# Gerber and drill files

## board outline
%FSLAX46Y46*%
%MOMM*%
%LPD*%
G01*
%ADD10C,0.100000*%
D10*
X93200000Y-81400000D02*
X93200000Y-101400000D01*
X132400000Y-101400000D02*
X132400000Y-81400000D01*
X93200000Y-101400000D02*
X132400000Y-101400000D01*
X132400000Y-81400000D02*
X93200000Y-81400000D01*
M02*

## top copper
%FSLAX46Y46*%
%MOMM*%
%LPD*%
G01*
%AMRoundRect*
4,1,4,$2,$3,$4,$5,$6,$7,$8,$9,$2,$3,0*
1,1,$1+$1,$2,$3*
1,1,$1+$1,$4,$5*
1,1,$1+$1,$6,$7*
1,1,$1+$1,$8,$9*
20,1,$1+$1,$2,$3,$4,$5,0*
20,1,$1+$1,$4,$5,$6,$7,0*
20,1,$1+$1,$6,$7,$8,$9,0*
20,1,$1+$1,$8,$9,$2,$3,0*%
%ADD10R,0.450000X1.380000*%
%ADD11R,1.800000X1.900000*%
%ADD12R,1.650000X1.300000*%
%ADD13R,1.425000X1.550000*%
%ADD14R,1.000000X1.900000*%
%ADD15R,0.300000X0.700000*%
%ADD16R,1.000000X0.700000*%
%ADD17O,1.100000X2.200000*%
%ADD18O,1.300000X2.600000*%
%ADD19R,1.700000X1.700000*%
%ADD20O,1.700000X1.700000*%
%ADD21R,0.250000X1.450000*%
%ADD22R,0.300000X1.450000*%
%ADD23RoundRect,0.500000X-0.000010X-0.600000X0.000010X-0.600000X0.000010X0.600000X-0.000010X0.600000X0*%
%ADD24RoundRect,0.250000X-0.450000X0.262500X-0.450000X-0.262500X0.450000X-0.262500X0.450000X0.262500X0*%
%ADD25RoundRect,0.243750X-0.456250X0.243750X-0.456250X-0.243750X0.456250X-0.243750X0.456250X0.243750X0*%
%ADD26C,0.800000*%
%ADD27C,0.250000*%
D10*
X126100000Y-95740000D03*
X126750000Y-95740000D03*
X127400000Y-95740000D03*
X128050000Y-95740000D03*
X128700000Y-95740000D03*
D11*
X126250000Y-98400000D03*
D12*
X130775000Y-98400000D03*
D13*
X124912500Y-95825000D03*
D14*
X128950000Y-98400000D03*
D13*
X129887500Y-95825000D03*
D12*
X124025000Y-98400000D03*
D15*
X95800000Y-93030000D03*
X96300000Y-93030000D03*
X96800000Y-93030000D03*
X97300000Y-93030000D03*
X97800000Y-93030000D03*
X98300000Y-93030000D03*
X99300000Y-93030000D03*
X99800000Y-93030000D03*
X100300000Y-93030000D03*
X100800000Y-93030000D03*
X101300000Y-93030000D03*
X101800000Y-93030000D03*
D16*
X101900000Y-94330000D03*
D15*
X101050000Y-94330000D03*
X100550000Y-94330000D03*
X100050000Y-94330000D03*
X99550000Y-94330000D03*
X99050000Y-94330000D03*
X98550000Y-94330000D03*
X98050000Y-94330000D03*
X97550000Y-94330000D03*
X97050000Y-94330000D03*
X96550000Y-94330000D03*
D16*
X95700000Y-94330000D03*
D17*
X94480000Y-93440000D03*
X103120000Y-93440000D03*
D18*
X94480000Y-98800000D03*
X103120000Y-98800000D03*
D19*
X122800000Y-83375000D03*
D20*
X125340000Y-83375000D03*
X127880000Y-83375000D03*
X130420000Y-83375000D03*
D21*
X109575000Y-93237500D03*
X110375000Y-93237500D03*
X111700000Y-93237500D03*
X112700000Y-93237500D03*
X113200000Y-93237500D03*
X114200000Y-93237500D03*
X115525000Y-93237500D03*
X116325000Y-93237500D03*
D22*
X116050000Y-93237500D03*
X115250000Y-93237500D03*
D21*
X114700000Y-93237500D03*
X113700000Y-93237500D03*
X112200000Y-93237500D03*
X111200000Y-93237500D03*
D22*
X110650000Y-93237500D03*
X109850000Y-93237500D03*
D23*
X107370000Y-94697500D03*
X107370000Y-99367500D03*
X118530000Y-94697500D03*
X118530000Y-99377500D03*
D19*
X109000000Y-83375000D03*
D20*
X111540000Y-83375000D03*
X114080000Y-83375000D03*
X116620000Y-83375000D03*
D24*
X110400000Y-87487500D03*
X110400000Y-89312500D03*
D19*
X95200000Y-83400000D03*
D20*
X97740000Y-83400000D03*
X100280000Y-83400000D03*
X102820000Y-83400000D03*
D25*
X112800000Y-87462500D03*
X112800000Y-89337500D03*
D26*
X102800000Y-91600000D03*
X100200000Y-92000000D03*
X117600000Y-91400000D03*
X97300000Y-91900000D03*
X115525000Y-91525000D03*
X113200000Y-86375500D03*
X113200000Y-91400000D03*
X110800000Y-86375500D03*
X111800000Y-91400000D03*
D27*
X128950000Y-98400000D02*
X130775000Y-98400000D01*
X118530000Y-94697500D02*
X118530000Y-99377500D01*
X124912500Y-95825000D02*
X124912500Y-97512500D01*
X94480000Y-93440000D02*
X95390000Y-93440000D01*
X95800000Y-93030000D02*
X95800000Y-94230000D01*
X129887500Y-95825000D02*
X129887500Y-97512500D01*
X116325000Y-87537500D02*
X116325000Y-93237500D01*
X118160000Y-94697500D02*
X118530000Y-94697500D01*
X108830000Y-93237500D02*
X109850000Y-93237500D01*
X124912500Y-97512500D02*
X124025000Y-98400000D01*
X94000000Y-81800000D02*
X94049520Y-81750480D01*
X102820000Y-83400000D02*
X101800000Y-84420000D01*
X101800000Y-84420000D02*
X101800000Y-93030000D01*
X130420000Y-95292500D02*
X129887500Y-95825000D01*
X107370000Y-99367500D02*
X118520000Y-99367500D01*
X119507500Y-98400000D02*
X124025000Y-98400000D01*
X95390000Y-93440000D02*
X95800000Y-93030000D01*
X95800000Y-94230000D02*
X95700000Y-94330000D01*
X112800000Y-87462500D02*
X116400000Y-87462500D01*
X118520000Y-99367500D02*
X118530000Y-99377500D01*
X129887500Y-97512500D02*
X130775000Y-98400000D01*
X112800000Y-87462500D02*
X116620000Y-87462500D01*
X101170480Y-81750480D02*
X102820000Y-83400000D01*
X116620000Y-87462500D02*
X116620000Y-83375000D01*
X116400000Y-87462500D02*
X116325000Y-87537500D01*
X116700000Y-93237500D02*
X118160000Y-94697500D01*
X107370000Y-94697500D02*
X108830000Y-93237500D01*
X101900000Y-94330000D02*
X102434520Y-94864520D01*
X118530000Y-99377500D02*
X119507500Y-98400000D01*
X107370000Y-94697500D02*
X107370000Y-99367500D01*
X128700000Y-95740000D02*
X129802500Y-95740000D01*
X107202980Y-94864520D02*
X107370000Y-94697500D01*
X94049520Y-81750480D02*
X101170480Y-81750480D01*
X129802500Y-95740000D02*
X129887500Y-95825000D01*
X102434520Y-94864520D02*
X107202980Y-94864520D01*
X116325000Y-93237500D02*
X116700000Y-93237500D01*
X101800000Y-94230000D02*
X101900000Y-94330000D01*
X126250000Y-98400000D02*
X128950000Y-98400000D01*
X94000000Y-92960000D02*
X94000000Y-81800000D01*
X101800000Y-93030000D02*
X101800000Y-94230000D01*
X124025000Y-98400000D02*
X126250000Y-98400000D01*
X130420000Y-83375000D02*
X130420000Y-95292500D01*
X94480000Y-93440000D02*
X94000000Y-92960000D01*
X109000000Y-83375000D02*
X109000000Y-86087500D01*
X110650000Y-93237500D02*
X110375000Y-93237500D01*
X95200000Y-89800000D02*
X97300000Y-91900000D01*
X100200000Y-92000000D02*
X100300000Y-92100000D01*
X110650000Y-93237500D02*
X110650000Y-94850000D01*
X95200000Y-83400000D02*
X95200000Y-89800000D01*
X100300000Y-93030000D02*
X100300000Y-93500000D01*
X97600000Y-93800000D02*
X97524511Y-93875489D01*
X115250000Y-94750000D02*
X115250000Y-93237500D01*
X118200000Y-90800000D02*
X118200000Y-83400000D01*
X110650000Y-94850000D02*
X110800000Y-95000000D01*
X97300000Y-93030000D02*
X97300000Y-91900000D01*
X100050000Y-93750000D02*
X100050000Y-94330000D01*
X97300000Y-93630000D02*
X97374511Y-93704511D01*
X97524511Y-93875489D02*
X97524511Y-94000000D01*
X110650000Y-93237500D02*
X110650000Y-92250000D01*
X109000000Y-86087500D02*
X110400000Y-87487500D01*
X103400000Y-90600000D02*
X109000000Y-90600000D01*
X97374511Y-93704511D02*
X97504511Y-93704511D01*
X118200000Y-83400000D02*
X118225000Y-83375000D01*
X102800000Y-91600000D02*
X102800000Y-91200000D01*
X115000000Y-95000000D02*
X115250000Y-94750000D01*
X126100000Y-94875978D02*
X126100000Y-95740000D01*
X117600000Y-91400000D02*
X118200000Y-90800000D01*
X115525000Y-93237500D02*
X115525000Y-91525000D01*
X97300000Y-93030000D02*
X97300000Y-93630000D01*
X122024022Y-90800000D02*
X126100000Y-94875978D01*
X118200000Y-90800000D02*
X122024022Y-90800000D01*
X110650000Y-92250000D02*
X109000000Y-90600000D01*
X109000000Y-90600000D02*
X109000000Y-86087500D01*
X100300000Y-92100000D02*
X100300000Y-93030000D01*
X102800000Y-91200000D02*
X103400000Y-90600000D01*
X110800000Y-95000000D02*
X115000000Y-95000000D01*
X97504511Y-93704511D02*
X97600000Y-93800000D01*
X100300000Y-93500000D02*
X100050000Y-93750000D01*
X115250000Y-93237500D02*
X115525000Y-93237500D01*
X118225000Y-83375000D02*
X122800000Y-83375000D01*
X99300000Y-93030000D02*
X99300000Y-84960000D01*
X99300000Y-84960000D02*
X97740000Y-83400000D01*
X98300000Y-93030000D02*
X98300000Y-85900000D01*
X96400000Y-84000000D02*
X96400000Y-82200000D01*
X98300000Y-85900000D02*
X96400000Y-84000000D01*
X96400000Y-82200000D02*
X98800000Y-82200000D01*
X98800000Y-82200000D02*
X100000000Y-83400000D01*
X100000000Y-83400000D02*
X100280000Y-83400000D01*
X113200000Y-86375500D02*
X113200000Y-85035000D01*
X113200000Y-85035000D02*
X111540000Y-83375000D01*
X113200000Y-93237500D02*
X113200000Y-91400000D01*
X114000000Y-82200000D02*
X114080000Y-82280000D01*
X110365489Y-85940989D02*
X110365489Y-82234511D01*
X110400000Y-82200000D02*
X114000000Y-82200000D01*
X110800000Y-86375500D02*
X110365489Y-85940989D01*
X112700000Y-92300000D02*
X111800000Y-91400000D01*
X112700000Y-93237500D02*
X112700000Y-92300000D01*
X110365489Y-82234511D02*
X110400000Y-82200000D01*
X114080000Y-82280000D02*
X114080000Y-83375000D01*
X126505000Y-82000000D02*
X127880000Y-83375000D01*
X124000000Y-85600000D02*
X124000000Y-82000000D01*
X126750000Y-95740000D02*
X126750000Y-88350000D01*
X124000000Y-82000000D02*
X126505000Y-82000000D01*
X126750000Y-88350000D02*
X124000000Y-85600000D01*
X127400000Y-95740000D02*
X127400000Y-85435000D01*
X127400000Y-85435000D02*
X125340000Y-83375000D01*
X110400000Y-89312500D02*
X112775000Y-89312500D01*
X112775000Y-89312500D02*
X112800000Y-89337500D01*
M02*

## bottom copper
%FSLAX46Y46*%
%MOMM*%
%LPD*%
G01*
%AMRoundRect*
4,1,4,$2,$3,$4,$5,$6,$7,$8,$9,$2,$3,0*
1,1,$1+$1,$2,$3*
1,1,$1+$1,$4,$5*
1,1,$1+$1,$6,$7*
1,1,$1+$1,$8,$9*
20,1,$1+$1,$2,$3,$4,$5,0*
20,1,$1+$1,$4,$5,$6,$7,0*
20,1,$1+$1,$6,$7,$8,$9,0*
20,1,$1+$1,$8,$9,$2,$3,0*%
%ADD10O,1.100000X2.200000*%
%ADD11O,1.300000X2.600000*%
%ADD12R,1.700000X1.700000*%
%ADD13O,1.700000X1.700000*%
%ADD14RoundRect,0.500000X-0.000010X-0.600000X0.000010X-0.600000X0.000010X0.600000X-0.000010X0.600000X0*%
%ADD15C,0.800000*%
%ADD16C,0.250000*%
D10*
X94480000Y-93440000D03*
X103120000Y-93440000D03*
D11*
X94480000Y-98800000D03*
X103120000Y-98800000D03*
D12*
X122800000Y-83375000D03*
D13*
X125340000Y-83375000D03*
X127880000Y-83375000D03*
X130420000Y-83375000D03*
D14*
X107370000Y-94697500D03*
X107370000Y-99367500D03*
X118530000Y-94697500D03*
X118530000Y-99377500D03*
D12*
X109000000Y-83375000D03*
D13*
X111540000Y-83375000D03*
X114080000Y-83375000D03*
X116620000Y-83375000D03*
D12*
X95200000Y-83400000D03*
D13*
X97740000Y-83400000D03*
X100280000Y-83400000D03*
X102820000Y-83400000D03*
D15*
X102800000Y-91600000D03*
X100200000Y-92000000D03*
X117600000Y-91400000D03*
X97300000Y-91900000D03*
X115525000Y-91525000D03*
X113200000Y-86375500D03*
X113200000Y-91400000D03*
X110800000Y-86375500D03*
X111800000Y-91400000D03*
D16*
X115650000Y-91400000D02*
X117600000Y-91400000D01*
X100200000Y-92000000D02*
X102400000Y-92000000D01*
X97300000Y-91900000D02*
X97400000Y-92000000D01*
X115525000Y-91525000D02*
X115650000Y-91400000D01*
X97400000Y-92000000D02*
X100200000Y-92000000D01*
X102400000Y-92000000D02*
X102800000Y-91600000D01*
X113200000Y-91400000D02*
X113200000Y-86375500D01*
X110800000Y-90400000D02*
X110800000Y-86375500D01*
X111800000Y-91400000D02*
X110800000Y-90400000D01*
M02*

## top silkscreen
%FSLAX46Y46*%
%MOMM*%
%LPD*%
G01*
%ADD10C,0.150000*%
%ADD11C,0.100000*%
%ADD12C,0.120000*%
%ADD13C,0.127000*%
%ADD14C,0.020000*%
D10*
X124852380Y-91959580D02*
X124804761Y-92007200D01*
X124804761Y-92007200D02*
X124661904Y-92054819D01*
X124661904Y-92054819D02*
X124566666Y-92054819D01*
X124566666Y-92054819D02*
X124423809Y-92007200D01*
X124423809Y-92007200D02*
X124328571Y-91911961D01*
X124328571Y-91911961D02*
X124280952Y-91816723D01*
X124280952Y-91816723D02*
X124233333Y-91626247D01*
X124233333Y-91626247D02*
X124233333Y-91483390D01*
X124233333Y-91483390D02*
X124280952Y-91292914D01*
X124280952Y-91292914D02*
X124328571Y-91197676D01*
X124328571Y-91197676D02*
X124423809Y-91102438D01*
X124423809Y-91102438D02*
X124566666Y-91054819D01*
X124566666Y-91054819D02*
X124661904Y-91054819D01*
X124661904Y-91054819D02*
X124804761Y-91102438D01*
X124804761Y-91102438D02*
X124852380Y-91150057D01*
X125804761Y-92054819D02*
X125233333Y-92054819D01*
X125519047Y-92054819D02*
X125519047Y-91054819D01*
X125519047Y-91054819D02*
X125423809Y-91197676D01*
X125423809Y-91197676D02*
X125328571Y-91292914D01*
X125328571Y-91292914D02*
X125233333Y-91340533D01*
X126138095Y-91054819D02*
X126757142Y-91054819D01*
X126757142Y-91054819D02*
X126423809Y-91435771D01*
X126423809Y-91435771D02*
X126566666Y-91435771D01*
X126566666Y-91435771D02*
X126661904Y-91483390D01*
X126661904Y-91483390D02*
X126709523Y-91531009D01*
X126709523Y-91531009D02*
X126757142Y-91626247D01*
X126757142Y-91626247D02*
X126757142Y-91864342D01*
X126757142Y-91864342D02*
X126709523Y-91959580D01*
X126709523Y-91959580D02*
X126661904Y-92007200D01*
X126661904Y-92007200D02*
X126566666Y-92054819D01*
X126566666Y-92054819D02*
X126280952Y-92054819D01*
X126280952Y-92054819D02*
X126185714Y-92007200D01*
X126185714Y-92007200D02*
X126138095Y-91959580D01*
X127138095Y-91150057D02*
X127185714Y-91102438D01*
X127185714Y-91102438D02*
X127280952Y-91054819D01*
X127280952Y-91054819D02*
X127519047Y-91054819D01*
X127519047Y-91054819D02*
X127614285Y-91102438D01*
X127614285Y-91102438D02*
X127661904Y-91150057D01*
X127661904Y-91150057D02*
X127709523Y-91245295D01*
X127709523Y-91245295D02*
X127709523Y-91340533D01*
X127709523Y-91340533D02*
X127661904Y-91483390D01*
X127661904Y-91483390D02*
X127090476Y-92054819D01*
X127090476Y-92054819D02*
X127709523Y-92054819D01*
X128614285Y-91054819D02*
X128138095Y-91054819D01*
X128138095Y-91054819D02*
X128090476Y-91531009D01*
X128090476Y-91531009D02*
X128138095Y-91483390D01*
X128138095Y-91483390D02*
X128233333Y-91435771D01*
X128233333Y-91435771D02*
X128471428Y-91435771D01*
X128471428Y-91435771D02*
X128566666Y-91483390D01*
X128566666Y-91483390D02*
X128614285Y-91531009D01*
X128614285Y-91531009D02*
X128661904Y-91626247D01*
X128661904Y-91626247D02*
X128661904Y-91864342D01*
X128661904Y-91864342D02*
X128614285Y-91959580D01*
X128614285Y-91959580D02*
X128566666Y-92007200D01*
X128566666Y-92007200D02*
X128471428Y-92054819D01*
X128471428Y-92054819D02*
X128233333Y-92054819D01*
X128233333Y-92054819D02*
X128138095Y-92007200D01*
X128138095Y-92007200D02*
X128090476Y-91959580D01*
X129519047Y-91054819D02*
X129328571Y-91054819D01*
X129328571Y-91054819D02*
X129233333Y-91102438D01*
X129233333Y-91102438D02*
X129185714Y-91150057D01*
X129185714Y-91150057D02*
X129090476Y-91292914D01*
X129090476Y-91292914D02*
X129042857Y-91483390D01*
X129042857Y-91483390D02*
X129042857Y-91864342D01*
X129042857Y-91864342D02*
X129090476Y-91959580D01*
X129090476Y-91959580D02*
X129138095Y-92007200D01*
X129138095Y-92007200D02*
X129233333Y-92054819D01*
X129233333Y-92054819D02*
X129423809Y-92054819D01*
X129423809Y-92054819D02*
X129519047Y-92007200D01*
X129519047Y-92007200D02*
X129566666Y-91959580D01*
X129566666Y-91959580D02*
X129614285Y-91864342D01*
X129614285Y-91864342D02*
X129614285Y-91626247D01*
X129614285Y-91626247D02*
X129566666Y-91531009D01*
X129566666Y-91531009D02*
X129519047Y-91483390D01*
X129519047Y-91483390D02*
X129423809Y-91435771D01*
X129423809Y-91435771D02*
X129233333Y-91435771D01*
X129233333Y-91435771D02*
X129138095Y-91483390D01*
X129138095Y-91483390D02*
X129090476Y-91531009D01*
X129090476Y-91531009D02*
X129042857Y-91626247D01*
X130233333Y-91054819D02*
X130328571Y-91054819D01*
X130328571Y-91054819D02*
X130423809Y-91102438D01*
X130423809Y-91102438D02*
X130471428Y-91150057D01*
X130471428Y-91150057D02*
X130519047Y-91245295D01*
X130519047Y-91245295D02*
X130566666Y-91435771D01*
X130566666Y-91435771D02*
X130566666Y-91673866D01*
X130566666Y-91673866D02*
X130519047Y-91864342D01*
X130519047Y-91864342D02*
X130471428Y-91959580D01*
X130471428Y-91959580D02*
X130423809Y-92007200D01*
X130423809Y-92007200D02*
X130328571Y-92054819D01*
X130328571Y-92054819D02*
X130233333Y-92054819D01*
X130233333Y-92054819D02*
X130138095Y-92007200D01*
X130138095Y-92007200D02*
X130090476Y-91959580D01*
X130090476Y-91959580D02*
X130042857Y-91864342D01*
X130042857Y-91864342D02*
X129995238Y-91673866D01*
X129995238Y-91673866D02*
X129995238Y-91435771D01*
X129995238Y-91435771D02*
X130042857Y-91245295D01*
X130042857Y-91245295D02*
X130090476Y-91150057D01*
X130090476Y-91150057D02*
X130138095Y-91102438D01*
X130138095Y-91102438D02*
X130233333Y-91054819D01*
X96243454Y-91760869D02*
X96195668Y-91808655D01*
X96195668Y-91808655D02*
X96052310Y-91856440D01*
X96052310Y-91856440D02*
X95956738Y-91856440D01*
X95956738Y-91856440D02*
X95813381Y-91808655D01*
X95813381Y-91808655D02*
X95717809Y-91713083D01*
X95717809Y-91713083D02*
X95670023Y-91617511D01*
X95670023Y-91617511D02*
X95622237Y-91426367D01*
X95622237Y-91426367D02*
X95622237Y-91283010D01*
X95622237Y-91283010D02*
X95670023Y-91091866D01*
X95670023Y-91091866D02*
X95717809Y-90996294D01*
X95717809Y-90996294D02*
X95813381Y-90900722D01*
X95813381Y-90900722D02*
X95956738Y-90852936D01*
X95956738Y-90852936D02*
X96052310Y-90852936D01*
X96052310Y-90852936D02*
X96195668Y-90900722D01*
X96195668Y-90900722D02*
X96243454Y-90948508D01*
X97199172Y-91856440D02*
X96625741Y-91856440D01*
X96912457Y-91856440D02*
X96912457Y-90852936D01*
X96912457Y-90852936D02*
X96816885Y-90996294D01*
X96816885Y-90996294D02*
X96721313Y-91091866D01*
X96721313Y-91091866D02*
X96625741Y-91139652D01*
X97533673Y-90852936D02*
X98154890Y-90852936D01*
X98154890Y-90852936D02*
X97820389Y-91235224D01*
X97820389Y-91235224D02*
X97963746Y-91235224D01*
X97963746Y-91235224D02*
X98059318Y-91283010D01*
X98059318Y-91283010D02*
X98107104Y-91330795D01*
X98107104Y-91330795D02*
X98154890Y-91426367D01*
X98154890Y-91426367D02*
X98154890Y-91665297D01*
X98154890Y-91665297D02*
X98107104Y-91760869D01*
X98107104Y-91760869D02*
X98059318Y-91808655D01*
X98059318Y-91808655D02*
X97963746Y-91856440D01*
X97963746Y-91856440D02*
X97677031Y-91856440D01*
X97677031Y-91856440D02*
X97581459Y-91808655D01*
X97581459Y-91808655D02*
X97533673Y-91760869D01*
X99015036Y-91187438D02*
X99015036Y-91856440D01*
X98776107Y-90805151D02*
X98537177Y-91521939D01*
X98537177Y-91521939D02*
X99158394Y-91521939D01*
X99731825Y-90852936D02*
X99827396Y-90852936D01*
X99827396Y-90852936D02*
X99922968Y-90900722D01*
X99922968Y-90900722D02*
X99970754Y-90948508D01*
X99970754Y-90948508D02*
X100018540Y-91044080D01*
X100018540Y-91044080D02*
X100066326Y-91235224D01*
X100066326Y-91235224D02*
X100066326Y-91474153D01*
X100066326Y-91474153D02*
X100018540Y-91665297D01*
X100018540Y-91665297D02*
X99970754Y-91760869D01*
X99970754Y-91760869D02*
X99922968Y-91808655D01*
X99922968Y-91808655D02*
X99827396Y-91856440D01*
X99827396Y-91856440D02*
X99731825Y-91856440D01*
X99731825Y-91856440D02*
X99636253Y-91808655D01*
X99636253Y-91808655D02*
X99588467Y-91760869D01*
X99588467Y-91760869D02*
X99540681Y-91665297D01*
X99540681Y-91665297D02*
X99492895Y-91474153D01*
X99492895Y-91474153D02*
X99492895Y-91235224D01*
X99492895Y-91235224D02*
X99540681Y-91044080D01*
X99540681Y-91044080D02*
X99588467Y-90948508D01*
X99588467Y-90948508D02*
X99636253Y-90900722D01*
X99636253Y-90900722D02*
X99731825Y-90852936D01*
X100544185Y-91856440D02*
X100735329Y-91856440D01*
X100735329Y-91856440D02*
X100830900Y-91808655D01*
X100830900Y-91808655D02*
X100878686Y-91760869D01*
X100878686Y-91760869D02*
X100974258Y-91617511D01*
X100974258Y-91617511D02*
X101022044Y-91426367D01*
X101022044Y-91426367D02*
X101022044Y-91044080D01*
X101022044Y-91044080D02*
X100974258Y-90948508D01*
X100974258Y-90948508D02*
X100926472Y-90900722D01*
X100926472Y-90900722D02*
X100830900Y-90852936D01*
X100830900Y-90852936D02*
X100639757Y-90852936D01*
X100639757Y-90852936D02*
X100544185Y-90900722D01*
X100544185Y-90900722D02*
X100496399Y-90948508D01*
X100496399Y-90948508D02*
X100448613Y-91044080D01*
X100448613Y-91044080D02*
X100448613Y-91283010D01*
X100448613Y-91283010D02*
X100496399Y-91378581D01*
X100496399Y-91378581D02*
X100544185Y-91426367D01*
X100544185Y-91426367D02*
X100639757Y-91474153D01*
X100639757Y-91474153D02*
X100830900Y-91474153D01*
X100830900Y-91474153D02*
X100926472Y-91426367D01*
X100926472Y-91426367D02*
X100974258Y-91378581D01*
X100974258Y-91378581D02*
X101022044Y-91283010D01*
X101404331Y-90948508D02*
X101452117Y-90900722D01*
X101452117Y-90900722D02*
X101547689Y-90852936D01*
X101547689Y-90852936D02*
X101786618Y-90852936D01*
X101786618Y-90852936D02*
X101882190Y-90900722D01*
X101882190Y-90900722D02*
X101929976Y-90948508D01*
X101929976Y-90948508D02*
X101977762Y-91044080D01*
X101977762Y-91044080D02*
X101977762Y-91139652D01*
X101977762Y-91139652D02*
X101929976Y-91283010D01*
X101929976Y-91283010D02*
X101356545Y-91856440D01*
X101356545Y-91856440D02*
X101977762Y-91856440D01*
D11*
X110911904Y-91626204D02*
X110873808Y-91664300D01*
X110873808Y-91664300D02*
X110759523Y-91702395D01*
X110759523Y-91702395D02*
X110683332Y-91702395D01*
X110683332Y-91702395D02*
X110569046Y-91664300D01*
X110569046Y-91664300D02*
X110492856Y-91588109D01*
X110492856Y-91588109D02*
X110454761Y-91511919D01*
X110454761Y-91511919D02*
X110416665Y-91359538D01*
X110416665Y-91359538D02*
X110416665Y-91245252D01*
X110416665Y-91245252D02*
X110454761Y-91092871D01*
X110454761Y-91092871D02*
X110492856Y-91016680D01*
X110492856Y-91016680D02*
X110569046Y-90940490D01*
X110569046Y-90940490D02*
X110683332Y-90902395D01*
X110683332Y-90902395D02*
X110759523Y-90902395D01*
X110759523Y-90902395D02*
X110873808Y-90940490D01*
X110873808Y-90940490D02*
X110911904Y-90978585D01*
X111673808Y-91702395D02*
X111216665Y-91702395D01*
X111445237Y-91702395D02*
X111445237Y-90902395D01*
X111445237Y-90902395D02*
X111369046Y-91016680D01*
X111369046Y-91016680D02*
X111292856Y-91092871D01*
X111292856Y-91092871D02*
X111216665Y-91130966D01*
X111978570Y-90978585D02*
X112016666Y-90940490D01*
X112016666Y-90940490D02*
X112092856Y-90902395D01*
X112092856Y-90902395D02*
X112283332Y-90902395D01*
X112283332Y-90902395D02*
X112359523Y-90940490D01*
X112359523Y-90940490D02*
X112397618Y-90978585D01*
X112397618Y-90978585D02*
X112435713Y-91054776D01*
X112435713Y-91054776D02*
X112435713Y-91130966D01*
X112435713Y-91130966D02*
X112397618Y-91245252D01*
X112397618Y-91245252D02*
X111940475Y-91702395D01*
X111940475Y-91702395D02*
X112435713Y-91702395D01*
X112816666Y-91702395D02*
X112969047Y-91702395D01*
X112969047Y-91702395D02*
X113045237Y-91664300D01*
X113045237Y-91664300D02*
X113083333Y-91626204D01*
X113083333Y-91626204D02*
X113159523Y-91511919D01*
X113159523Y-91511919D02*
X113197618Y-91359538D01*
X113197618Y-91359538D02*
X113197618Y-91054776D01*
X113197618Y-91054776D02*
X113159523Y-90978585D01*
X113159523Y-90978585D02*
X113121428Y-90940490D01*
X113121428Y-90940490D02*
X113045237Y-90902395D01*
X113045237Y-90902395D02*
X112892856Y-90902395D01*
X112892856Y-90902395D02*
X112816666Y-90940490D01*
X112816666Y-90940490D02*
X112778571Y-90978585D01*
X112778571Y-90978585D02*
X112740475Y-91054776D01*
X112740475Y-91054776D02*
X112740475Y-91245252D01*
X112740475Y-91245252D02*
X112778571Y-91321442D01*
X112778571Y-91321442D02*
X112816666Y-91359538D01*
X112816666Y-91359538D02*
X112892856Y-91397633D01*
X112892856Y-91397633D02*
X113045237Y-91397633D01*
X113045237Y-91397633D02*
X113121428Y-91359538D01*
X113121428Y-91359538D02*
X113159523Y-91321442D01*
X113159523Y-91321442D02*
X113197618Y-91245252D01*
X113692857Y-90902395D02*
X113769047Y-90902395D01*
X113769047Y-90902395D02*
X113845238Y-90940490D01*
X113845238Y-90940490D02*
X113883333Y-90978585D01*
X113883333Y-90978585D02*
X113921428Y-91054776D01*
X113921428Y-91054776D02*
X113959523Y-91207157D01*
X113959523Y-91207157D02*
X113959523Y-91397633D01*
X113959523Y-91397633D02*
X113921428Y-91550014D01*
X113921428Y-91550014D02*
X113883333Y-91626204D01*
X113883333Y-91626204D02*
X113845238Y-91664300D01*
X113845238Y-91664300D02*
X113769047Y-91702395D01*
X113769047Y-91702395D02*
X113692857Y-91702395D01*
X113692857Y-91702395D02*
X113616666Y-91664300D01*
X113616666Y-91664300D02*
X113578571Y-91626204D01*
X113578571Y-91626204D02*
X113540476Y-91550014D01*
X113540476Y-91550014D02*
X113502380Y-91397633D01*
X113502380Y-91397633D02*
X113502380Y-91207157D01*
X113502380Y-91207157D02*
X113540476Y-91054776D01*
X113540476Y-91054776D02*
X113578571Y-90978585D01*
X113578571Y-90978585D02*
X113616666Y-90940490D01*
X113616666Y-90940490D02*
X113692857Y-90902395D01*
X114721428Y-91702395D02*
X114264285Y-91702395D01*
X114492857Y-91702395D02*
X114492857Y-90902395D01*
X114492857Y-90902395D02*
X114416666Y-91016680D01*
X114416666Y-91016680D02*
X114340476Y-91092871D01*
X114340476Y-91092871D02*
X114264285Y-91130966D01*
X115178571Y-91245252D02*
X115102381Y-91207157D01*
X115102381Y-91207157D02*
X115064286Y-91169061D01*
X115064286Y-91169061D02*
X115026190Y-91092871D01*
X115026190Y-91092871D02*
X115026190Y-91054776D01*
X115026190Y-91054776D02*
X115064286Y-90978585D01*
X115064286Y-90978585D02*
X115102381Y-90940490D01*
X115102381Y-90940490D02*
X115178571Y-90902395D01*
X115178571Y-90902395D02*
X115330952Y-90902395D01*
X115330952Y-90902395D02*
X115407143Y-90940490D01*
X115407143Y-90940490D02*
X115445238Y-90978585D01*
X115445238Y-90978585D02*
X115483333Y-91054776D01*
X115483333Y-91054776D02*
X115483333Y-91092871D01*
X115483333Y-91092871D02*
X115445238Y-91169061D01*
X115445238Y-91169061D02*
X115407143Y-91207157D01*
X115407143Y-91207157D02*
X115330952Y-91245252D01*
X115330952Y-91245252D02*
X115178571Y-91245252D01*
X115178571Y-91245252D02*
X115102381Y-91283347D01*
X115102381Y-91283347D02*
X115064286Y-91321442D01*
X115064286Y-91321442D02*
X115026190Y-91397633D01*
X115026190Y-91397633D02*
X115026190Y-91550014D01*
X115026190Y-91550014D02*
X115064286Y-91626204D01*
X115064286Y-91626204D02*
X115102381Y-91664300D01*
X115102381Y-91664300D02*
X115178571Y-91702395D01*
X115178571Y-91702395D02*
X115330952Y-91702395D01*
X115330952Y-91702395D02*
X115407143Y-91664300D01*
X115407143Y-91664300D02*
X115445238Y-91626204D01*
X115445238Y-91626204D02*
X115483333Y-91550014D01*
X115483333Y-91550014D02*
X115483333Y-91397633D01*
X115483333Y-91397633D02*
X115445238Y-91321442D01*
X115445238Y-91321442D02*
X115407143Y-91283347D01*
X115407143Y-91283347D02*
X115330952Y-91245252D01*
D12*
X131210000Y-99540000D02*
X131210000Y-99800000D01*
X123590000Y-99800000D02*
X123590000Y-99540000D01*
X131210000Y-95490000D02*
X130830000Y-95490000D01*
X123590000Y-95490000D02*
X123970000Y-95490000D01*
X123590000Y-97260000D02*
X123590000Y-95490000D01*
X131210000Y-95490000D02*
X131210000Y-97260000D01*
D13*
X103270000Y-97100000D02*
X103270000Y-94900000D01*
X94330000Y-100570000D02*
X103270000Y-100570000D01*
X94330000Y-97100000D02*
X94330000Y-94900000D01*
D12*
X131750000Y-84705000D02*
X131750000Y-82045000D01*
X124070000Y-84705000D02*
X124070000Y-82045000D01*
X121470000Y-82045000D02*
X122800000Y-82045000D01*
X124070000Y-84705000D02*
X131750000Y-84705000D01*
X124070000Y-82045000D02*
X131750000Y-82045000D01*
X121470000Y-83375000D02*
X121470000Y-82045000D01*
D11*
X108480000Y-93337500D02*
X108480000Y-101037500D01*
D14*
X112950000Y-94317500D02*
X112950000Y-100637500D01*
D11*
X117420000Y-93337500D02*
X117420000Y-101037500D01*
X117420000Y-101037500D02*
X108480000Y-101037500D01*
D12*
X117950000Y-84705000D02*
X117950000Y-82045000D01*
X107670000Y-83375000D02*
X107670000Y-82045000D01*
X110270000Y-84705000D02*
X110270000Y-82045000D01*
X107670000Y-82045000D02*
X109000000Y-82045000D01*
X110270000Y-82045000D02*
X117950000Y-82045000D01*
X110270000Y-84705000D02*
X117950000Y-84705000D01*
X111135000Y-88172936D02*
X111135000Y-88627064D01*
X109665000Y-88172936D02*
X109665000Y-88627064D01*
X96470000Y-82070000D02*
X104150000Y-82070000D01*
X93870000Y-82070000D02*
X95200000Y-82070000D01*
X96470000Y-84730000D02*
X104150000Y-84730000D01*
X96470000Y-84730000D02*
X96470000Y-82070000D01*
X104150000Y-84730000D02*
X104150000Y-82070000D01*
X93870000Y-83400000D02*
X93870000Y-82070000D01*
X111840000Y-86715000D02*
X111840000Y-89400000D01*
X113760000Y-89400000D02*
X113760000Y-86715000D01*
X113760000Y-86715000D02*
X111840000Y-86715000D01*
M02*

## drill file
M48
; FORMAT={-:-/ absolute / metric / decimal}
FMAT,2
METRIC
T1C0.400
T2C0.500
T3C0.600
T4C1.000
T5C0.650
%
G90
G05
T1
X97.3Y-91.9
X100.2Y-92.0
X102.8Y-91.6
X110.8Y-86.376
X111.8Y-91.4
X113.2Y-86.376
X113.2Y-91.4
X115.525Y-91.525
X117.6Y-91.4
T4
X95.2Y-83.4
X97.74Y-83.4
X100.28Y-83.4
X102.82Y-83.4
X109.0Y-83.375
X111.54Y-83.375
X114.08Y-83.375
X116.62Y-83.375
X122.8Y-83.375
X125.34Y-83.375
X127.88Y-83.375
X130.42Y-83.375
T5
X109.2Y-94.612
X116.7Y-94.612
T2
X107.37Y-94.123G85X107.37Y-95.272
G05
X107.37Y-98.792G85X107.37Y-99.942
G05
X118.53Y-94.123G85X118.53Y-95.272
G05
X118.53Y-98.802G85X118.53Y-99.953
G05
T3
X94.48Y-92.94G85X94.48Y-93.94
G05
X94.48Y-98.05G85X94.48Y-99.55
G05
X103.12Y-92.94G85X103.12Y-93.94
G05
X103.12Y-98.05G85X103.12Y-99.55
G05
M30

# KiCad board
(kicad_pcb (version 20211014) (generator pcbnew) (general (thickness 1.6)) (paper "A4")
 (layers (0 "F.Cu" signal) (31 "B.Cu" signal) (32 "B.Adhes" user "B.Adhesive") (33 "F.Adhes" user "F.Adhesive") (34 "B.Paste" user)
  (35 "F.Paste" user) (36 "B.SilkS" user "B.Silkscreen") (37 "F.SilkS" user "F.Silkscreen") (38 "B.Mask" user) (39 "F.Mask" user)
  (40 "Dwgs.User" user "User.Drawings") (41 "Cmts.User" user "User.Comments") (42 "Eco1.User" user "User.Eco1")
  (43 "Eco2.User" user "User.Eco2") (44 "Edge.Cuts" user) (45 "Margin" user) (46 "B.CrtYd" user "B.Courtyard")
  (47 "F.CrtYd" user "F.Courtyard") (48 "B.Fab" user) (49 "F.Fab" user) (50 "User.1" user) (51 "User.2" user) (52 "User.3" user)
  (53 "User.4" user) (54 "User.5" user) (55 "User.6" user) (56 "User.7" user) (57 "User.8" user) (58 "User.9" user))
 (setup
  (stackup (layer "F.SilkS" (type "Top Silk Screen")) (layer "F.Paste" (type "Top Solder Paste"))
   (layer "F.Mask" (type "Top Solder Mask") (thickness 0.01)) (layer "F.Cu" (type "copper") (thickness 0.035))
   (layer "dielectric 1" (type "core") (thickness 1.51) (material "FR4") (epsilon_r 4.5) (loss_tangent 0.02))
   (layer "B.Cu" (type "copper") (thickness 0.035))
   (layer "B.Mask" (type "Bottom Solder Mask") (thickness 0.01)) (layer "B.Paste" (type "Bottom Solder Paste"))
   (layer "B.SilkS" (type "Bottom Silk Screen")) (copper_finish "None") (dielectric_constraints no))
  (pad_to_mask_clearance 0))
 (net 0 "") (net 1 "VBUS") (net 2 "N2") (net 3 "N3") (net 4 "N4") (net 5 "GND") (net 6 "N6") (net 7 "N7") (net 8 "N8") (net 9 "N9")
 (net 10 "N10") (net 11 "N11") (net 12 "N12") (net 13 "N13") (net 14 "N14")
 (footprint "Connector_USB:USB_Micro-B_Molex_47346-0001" (layer "F.Cu") (at 127.4 97.2)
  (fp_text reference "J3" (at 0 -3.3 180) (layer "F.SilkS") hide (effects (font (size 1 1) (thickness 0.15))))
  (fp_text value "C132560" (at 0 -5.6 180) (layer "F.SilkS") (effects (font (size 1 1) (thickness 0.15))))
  (fp_line (start 3.81 2.34) (end 3.81 2.6) (layer "F.SilkS") (width 0.12))
  (fp_line (start -3.81 2.6) (end -3.81 2.34) (layer "F.SilkS") (width 0.12))
  (fp_line (start 3.81 -1.71) (end 3.43 -1.71) (layer "F.SilkS") (width 0.12))
  (fp_line (start -3.81 -1.71) (end -3.43 -1.71) (layer "F.SilkS") (width 0.12))
  (fp_line (start -3.81 0.06) (end -3.81 -1.71) (layer "F.SilkS") (width 0.12))
  (fp_line (start 3.81 -1.71) (end 3.81 0.06) (layer "F.SilkS") (width 0.12))
  (pad "1" smd rect locked (at -1.3 -1.46) (size 0.45 1.38) (layers "F.Cu" "F.Paste" "F.Mask") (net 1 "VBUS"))
  (pad "2" smd rect locked (at -0.65 -1.46) (size 0.45 1.38) (layers "F.Cu" "F.Paste" "F.Mask") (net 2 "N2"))
  (pad "3" smd rect locked (at 0 -1.46) (size 0.45 1.38) (layers "F.Cu" "F.Paste" "F.Mask") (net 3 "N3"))
  (pad "4" smd rect locked (at 0.65 -1.46) (size 0.45 1.38) (layers "F.Cu" "F.Paste" "F.Mask") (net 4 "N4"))
  (pad "5" smd rect locked (at 1.3 -1.46) (size 0.45 1.38) (layers "F.Cu" "F.Paste" "F.Mask") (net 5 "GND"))
  (pad "6" smd rect locked (at -1.15 1.2) (size 1.8 1.9) (layers "F.Cu" "F.Paste" "F.Mask") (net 5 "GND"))
  (pad "6" smd rect locked (at 3.375 1.2) (size 1.65 1.3) (layers "F.Cu" "F.Paste" "F.Mask") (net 5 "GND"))
  (pad "6" smd rect locked (at -2.4875 -1.375) (size 1.425 1.55) (layers "F.Cu" "F.Paste" "F.Mask") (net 5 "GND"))
  (pad "6" smd rect locked (at 1.55 1.2) (size 1 1.9) (layers "F.Cu" "F.Paste" "F.Mask") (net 5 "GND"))
  (pad "6" smd rect locked (at 2.4875 -1.375) (size 1.425 1.55) (layers "F.Cu" "F.Paste" "F.Mask") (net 5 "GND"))
  (pad "6" smd rect locked (at -3.375 1.2) (size 1.65 1.3) (layers "F.Cu" "F.Paste" "F.Mask") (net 5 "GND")))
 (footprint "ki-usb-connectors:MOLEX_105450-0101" (layer "F.Cu") (at 98.8 96.8)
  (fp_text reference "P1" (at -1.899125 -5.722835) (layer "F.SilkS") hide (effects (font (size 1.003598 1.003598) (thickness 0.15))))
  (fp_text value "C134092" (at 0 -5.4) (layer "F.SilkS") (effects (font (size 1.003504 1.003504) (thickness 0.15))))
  (fp_line (start 4.47 0.3) (end 4.47 -1.9) (layer "F.SilkS") (width 0.127))
  (fp_line (start -4.47 3.77) (end 4.47 3.77) (layer "F.SilkS") (width 0.127))
  (fp_line (start -4.47 0.3) (end -4.47 -1.9) (layer "F.SilkS") (width 0.127))
  (pad "A1" smd rect (at -3 -3.77) (size 0.3 0.7) (layers "F.Cu" "F.Paste" "F.Mask") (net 5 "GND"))
  (pad "A2" smd rect (at -2.5 -3.77) (size 0.3 0.7) (layers "F.Cu" "F.Paste" "F.Mask"))
  (pad "A3" smd rect (at -2 -3.77) (size 0.3 0.7) (layers "F.Cu" "F.Paste" "F.Mask"))
  (pad "A4" smd rect (at -1.5 -3.77) (size 0.3 0.7) (layers "F.Cu" "F.Paste" "F.Mask") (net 1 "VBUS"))
  (pad "A5" smd rect (at -1 -3.77) (size 0.3 0.7) (layers "F.Cu" "F.Paste" "F.Mask") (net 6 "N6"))
  (pad "A6" smd rect (at -0.5 -3.77) (size 0.3 0.7) (layers "F.Cu" "F.Paste" "F.Mask") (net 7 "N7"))
  (pad "A7" smd rect (at 0.5 -3.77) (size 0.3 0.7) (layers "F.Cu" "F.Paste" "F.Mask") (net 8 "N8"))
  (pad "A8" smd rect (at 1 -3.77) (size 0.3 0.7) (layers "F.Cu" "F.Paste" "F.Mask"))
  (pad "A9" smd rect (at 1.5 -3.77) (size 0.3 0.7) (layers "F.Cu" "F.Paste" "F.Mask") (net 1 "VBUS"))
  (pad "A10" smd rect (at 2 -3.77) (size 0.3 0.7) (layers "F.Cu" "F.Paste" "F.Mask"))
  (pad "A11" smd rect (at 2.5 -3.77) (size 0.3 0.7) (layers "F.Cu" "F.Paste" "F.Mask"))
  (pad "A12" smd rect (at 3 -3.77) (size 0.3 0.7) (layers "F.Cu" "F.Paste" "F.Mask") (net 5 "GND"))
  (pad "B1" smd rect (at 3.1 -2.47) (size 1 0.7) (layers "F.Cu" "F.Paste" "F.Mask") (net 5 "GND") (clearance 0.15))
  (pad "B2" smd rect (at 2.25 -2.47) (size 0.3 0.7) (layers "F.Cu" "F.Paste" "F.Mask"))
  (pad "B3" smd rect (at 1.75 -2.47) (size 0.3 0.7) (layers "F.Cu" "F.Paste" "F.Mask"))
  (pad "B4" smd rect (at 1.25 -2.47) (size 0.3 0.7) (layers "F.Cu" "F.Paste" "F.Mask") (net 1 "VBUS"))
  (pad "B5" smd rect (at 0.75 -2.47) (size 0.3 0.7) (layers "F.Cu" "F.Paste" "F.Mask") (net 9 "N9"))
  (pad "B6" smd rect (at 0.25 -2.47) (size 0.3 0.7) (layers "F.Cu" "F.Paste" "F.Mask"))
  (pad "B7" smd rect (at -0.25 -2.47) (size 0.3 0.7) (layers "F.Cu" "F.Paste" "F.Mask"))
  (pad "B8" smd rect (at -0.75 -2.47) (size 0.3 0.7) (layers "F.Cu" "F.Paste" "F.Mask"))
  (pad "B9" smd rect (at -1.25 -2.47) (size 0.3 0.7) (layers "F.Cu" "F.Paste" "F.Mask") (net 1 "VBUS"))
  (pad "B10" smd rect (at -1.75 -2.47) (size 0.3 0.7) (layers "F.Cu" "F.Paste" "F.Mask"))
  (pad "B11" smd rect (at -2.25 -2.47) (size 0.3 0.7) (layers "F.Cu" "F.Paste" "F.Mask"))
  (pad "B12" smd rect (at -3.1 -2.47) (size 1 0.7) (layers "F.Cu" "F.Paste" "F.Mask") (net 5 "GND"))
  (pad "S1" thru_hole oval (at -4.32 -3.36) (size 1.1 2.2) (drill oval 0.6 1.6) (layers *.Cu *.Mask) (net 5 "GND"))
  (pad "S2" thru_hole oval (at 4.32 -3.36) (size 1.1 2.2) (drill oval 0.6 1.6) (layers *.Cu *.Mask))
  (pad "S3" thru_hole oval (at -4.32 2) (size 1.3 2.6) (drill oval 0.6 2.1) (layers *.Cu *.Mask))
  (pad "S4" thru_hole oval (at 4.32 2) (size 1.3 2.6) (drill oval 0.6 2.1) (layers *.Cu *.Mask))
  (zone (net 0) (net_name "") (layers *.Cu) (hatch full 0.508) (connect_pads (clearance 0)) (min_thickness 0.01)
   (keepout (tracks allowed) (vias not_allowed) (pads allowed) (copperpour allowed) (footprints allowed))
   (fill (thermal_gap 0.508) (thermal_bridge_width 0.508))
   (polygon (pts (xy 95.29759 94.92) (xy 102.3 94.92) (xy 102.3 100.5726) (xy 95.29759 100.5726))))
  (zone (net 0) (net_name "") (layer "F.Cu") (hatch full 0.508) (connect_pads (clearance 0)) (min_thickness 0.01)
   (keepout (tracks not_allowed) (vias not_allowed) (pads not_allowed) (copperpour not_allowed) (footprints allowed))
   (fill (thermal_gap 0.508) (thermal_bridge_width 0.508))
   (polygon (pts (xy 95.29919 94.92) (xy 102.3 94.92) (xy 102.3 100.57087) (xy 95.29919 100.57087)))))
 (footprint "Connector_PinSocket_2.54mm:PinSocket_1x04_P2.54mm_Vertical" (layer "F.Cu") (at 122.8 83.375 90)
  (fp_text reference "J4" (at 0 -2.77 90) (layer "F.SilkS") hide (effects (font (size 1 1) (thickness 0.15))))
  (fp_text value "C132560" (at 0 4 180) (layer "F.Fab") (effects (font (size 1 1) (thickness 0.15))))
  (fp_line (start -1.33 8.95) (end 1.33 8.95) (layer "F.SilkS") (width 0.12))
  (fp_line (start -1.33 1.27) (end 1.33 1.27) (layer "F.SilkS") (width 0.12))
  (fp_line (start 1.33 -1.33) (end 1.33 0) (layer "F.SilkS") (width 0.12))
  (fp_line (start -1.33 1.27) (end -1.33 8.95) (layer "F.SilkS") (width 0.12))
  (fp_line (start 1.33 1.27) (end 1.33 8.95) (layer "F.SilkS") (width 0.12))
  (fp_line (start 0 -1.33) (end 1.33 -1.33) (layer "F.SilkS") (width 0.12))
  (pad "1" thru_hole rect locked (at 0 0 90) (size 1.7 1.7) (drill 1) (layers *.Cu *.Mask) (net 1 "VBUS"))
  (pad "2" thru_hole oval locked (at 0 2.54 90) (size 1.7 1.7) (drill 1) (layers *.Cu *.Mask) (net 3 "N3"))
  (pad "3" thru_hole oval locked (at 0 5.08 90) (size 1.7 1.7) (drill 1) (layers *.Cu *.Mask) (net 2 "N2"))
  (pad "4" thru_hole oval locked (at 0 7.62 90) (size 1.7 1.7) (drill 1) (layers *.Cu *.Mask) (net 5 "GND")))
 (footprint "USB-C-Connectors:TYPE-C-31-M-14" (layer "F.Cu") (at 112.95 98.3375)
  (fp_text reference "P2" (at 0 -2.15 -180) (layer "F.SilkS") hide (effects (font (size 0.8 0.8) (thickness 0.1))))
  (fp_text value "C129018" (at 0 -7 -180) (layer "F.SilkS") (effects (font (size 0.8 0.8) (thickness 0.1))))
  (fp_line (start -4.47 -5) (end -4.47 2.7) (layer "F.SilkS") (width 0.1))
  (fp_line (start 0 -4.02) (end 0 2.3) (layer "F.SilkS") (width 0.02))
  (fp_line (start 4.47 -5) (end 4.47 2.7) (layer "F.SilkS") (width 0.1))
  (fp_line (start 4.47 2.7) (end -4.47 2.7) (layer "F.SilkS") (width 0.1))
  (pad "" np_thru_hole circle (at 3.75 -3.725) (size 0.65 0.65) (drill 0.65) (layers *.Cu *.Mask) (solder_mask_margin 0.01)
   (solder_paste_margin 0.01) (clearance 0.01))
  (pad "" np_thru_hole circle (at -3.75 -3.725) (size 0.65 0.65) (drill 0.65) (layers *.Cu *.Mask) (solder_mask_margin 0.01)
   (solder_paste_margin 0.01) (clearance 0.01))
  (pad "A1" smd rect (at -3.375 -5.1) (size 0.25 1.45) (layers "F.Cu" "F.Paste" "F.Mask") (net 5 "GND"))
  (pad "A4" smd rect (at -2.575 -5.1) (size 0.25 1.45) (layers "F.Cu" "F.Paste" "F.Mask") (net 1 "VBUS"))
  (pad "A5" smd rect (at -1.25 -5.1) (size 0.25 1.45) (layers "F.Cu" "F.Paste" "F.Mask") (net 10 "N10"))
  (pad "A6" smd rect (at -0.25 -5.1) (size 0.25 1.45) (layers "F.Cu" "F.Paste" "F.Mask") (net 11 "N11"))
  (pad "A7" smd rect (at 0.25 -5.1) (size 0.25 1.45) (layers "F.Cu" "F.Paste" "F.Mask") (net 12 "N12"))
  (pad "A8" smd rect (at 1.25 -5.1) (size 0.25 1.45) (layers "F.Cu" "F.Paste" "F.Mask"))
  (pad "A9" smd rect (at 2.575 -5.1) (size 0.25 1.45) (layers "F.Cu" "F.Paste" "F.Mask") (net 1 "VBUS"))
  (pad "A12" smd rect (at 3.375 -5.1) (size 0.25 1.45) (layers "F.Cu" "F.Paste" "F.Mask") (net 5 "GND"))
  (pad "B1" smd rect (at 3.1 -5.1) (size 0.3 1.45) (layers "F.Cu" "F.Paste" "F.Mask") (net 5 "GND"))
  (pad "B4" smd rect (at 2.3 -5.1) (size 0.3 1.45) (layers "F.Cu" "F.Paste" "F.Mask") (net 1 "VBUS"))
  (pad "B5" smd rect (at 1.75 -5.1) (size 0.25 1.45) (layers "F.Cu" "F.Paste" "F.Mask") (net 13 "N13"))
  (pad "B6" smd rect (at 0.75 -5.1) (size 0.25 1.45) (layers "F.Cu" "F.Paste" "F.Mask"))
  (pad "B7" smd rect (at -0.75 -5.1) (size 0.25 1.45) (layers "F.Cu" "F.Paste" "F.Mask"))
  (pad "B8" smd rect (at -1.75 -5.1) (size 0.25 1.45) (layers "F.Cu" "F.Paste" "F.Mask"))
  (pad "B9" smd rect (at -2.3 -5.1) (size 0.3 1.45) (layers "F.Cu" "F.Paste" "F.Mask") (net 1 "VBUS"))
  (pad "B12" smd rect (at -3.1 -5.1) (size 0.3 1.45) (layers "F.Cu" "F.Paste" "F.Mask") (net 5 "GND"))
  (pad "S1" thru_hole roundrect (at -5.58 -3.64) (size 1 2.2) (drill oval 0.5 1.65) (layers *.Cu *.Mask) (roundrect_rratio 0.5)
   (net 5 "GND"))
  (pad "S1" thru_hole roundrect (at -5.58 1.03) (size 1 2.2) (drill oval 0.5 1.65) (layers *.Cu *.Mask) (roundrect_rratio 0.5) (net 5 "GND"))
  (pad "S1" thru_hole roundrect (at 5.58 -3.64) (size 1 2.2) (drill oval 0.5 1.65) (layers *.Cu *.Mask) (roundrect_rratio 0.5) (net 5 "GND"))
  (pad "S1" thru_hole roundrect (at 5.58 1.04) (size 1 2.2) (drill oval 0.5 1.65) (layers *.Cu *.Mask) (roundrect_rratio 0.5) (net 5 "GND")))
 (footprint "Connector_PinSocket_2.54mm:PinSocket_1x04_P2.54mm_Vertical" (layer "F.Cu") (at 109 83.375 90)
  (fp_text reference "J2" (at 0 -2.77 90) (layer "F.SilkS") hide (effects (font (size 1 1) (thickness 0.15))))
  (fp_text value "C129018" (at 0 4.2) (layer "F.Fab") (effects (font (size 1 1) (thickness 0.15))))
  (fp_line (start -1.33 8.95) (end 1.33 8.95) (layer "F.SilkS") (width 0.12))
  (fp_line (start 0 -1.33) (end 1.33 -1.33) (layer "F.SilkS") (width 0.12))
  (fp_line (start -1.33 1.27) (end 1.33 1.27) (layer "F.SilkS") (width 0.12))
  (fp_line (start 1.33 -1.33) (end 1.33 0) (layer "F.SilkS") (width 0.12))
  (fp_line (start 1.33 1.27) (end 1.33 8.95) (layer "F.SilkS") (width 0.12))
  (fp_line (start -1.33 1.27) (end -1.33 8.95) (layer "F.SilkS") (width 0.12))
  (pad "1" thru_hole rect locked (at 0 0 90) (size 1.7 1.7) (drill 1) (layers *.Cu *.Mask) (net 1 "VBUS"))
  (pad "2" thru_hole oval locked (at 0 2.54 90) (size 1.7 1.7) (drill 1) (layers *.Cu *.Mask) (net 12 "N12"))
  (pad "3" thru_hole oval locked (at 0 5.08 90) (size 1.7 1.7) (drill 1) (layers *.Cu *.Mask) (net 11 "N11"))
  (pad "4" thru_hole oval locked (at 0 7.62 90) (size 1.7 1.7) (drill 1) (layers *.Cu *.Mask) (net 5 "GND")))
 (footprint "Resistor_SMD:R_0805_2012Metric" (layer "F.Cu") (at 110.4 88.4 -90)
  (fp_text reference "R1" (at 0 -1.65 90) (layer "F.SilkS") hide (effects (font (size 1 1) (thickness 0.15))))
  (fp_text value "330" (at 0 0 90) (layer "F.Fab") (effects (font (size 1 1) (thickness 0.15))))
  (fp_line (start -0.227064 -0.735) (end 0.227064 -0.735) (layer "F.SilkS") (width 0.12))
  (fp_line (start -0.227064 0.735) (end 0.227064 0.735) (layer "F.SilkS") (width 0.12))
  (pad "1" smd roundrect locked (at -0.9125 0 270) (size 1.025 1.4) (layers "F.Cu" "F.Paste" "F.Mask") (roundrect_rratio 0.243902)
   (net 1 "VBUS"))
  (pad "2" smd roundrect locked (at 0.9125 0 270) (size 1.025 1.4) (layers "F.Cu" "F.Paste" "F.Mask") (roundrect_rratio 0.243902)
   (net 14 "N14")))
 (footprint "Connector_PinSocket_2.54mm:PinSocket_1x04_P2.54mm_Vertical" (layer "F.Cu") (at 95.2 83.4 90)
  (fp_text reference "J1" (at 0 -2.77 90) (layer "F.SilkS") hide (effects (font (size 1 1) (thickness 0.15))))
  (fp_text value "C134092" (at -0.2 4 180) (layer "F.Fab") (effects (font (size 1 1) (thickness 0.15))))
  (fp_line (start 1.33 1.27) (end 1.33 8.95) (layer "F.SilkS") (width 0.12))
  (fp_line (start 1.33 -1.33) (end 1.33 0) (layer "F.SilkS") (width 0.12))
  (fp_line (start -1.33 1.27) (end -1.33 8.95) (layer "F.SilkS") (width 0.12))
  (fp_line (start -1.33 1.27) (end 1.33 1.27) (layer "F.SilkS") (width 0.12))
  (fp_line (start -1.33 8.95) (end 1.33 8.95) (layer "F.SilkS") (width 0.12))
  (fp_line (start 0 -1.33) (end 1.33 -1.33) (layer "F.SilkS") (width 0.12))
  (pad "1" thru_hole rect locked (at 0 0 90) (size 1.7 1.7) (drill 1) (layers *.Cu *.Mask) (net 1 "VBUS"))
  (pad "2" thru_hole oval locked (at 0 2.54 90) (size 1.7 1.7) (drill 1) (layers *.Cu *.Mask) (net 8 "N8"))
  (pad "3" thru_hole oval locked (at 0 5.08 90) (size 1.7 1.7) (drill 1) (layers *.Cu *.Mask) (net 7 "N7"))
  (pad "4" thru_hole oval locked (at 0 7.62 90) (size 1.7 1.7) (drill 1) (layers *.Cu *.Mask) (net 5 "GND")))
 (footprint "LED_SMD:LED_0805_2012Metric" (layer "F.Cu") (at 112.8 88.4 -90)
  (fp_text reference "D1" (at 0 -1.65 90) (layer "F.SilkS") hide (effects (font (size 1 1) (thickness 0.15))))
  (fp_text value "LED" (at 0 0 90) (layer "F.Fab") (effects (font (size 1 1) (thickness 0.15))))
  (fp_line (start -1.685 0.96) (end 1 0.96) (layer "F.SilkS") (width 0.12))
  (fp_line (start 1 -0.96) (end -1.685 -0.96) (layer "F.SilkS") (width 0.12))
  (fp_line (start -1.685 -0.96) (end -1.685 0.96) (layer "F.SilkS") (width 0.12))
  (pad "1" smd roundrect locked (at -0.9375 0 270) (size 0.975 1.4) (layers "F.Cu" "F.Paste" "F.Mask") (roundrect_rratio 0.25) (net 5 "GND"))
  (pad "2" smd roundrect locked (at 0.9375 0 270) (size 0.975 1.4) (layers "F.Cu" "F.Paste" "F.Mask") (roundrect_rratio 0.25) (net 14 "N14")))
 (gr_line (start 93.2 81.4) (end 93.2 101.4) (layer "Edge.Cuts") (width 0.1))
 (gr_line (start 132.4 101.4) (end 132.4 81.4) (layer "Edge.Cuts") (width 0.1))
 (gr_line (start 93.2 101.4) (end 132.4 101.4) (layer "Edge.Cuts") (width 0.1))
 (gr_line (start 132.4 81.4) (end 93.2 81.4) (layer "Edge.Cuts") (width 0.1))
 (segment (start 128.95 98.4) (end 130.775 98.4) (width 0.25) (layer "F.Cu") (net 5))
 (segment (start 118.53 94.6975) (end 118.53 99.3775) (width 0.25) (layer "F.Cu") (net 5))
 (segment (start 124.9125 95.825) (end 124.9125 97.5125) (width 0.25) (layer "F.Cu") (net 5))
 (segment (start 94.48 93.44) (end 95.39 93.44) (width 0.25) (layer "F.Cu") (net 5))
 (segment (start 95.8 93.03) (end 95.8 94.23) (width 0.25) (layer "F.Cu") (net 5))
 (segment (start 129.8875 95.825) (end 129.8875 97.5125) (width 0.25) (layer "F.Cu") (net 5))
 (segment (start 116.325 87.5375) (end 116.325 93.2375) (width 0.25) (layer "F.Cu") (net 5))
 (segment (start 118.16 94.6975) (end 118.53 94.6975) (width 0.25) (layer "F.Cu") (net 5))
 (segment (start 108.83 93.2375) (end 109.85 93.2375) (width 0.25) (layer "F.Cu") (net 5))
 (segment (start 124.9125 97.5125) (end 124.025 98.4) (width 0.25) (layer "F.Cu") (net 5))
 (segment (start 94 81.8) (end 94.04952 81.75048) (width 0.25) (layer "F.Cu") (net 5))
 (segment (start 102.82 83.4) (end 101.8 84.42) (width 0.25) (layer "F.Cu") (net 5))
 (segment (start 101.8 84.42) (end 101.8 93.03) (width 0.25) (layer "F.Cu") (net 5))
 (segment (start 130.42 95.2925) (end 129.8875 95.825) (width 0.25) (layer "F.Cu") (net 5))
 (segment (start 107.37 99.3675) (end 118.52 99.3675) (width 0.25) (layer "F.Cu") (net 5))
 (segment (start 119.5075 98.4) (end 124.025 98.4) (width 0.25) (layer "F.Cu") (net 5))
 (segment (start 95.39 93.44) (end 95.8 93.03) (width 0.25) (layer "F.Cu") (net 5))
 (segment (start 95.8 94.23) (end 95.7 94.33) (width 0.25) (layer "F.Cu") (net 5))
 (segment (start 112.8 87.4625) (end 116.4 87.4625) (width 0.25) (layer "F.Cu") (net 5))
 (segment (start 118.52 99.3675) (end 118.53 99.3775) (width 0.25) (layer "F.Cu") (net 5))
 (segment (start 129.8875 97.5125) (end 130.775 98.4) (width 0.25) (layer "F.Cu") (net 5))
 (segment (start 112.8 87.4625) (end 116.62 87.4625) (width 0.25) (layer "F.Cu") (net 5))
 (segment (start 101.17048 81.75048) (end 102.82 83.4) (width 0.25) (layer "F.Cu") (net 5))
 (segment (start 116.62 87.4625) (end 116.62 83.375) (width 0.25) (layer "F.Cu") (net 5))
 (segment (start 116.4 87.4625) (end 116.325 87.5375) (width 0.25) (layer "F.Cu") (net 5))
 (segment (start 116.7 93.2375) (end 118.16 94.6975) (width 0.25) (layer "F.Cu") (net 5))
 (segment (start 107.37 94.6975) (end 108.83 93.2375) (width 0.25) (layer "F.Cu") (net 5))
 (segment (start 101.9 94.33) (end 102.43452 94.86452) (width 0.25) (layer "F.Cu") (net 5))
 (segment (start 118.53 99.3775) (end 119.5075 98.4) (width 0.25) (layer "F.Cu") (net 5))
 (segment (start 107.37 94.6975) (end 107.37 99.3675) (width 0.25) (layer "F.Cu") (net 5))
 (segment (start 128.7 95.74) (end 129.8025 95.74) (width 0.25) (layer "F.Cu") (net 5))
 (segment (start 107.20298 94.86452) (end 107.37 94.6975) (width 0.25) (layer "F.Cu") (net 5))
 (segment (start 94.04952 81.75048) (end 101.17048 81.75048) (width 0.25) (layer "F.Cu") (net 5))
 (segment (start 129.8025 95.74) (end 129.8875 95.825) (width 0.25) (layer "F.Cu") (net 5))
 (segment (start 102.43452 94.86452) (end 107.20298 94.86452) (width 0.25) (layer "F.Cu") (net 5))
 (segment (start 116.325 93.2375) (end 116.7 93.2375) (width 0.25) (layer "F.Cu") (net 5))
 (segment (start 101.8 94.23) (end 101.9 94.33) (width 0.25) (layer "F.Cu") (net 5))
 (segment (start 126.25 98.4) (end 128.95 98.4) (width 0.25) (layer "F.Cu") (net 5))
 (segment (start 94 92.96) (end 94 81.8) (width 0.25) (layer "F.Cu") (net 5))
 (segment (start 101.8 93.03) (end 101.8 94.23) (width 0.25) (layer "F.Cu") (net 5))
 (segment (start 124.025 98.4) (end 126.25 98.4) (width 0.25) (layer "F.Cu") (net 5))
 (segment (start 130.42 83.375) (end 130.42 95.2925) (width 0.25) (layer "F.Cu") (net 5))
 (segment (start 94.48 93.44) (end 94 92.96) (width 0.25) (layer "F.Cu") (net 5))
 (segment (start 109 83.375) (end 109 86.0875) (width 0.25) (layer "F.Cu") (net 1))
 (segment (start 110.65 93.2375) (end 110.375 93.2375) (width 0.25) (layer "F.Cu") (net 1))
 (segment (start 95.2 89.8) (end 97.3 91.9) (width 0.25) (layer "F.Cu") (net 1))
 (segment (start 100.2 92) (end 100.3 92.1) (width 0.25) (layer "F.Cu") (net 1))
 (segment (start 110.65 93.2375) (end 110.65 94.85) (width 0.25) (layer "F.Cu") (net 1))
 (segment (start 95.2 83.4) (end 95.2 89.8) (width 0.25) (layer "F.Cu") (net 1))
 (segment (start 100.3 93.03) (end 100.3 93.5) (width 0.25) (layer "F.Cu") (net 1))
 (segment (start 97.6 93.8) (end 97.524511 93.875489) (width 0.25) (layer "F.Cu") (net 1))
 (segment (start 115.25 94.75) (end 115.25 93.2375) (width 0.25) (layer "F.Cu") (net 1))
 (segment (start 118.2 90.8) (end 118.2 83.4) (width 0.25) (layer "F.Cu") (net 1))
 (segment (start 110.65 94.85) (end 110.8 95) (width 0.25) (layer "F.Cu") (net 1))
 (segment (start 97.3 93.03) (end 97.3 91.9) (width 0.25) (layer "F.Cu") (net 1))
 (segment (start 100.05 93.75) (end 100.05 94.33) (width 0.25) (layer "F.Cu") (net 1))
 (segment (start 97.3 93.63) (end 97.374511 93.704511) (width 0.25) (layer "F.Cu") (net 1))
 (segment (start 97.524511 93.875489) (end 97.524511 94) (width 0.25) (layer "F.Cu") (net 1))
 (segment (start 110.65 93.2375) (end 110.65 92.25) (width 0.25) (layer "F.Cu") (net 1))
 (segment (start 109 86.0875) (end 110.4 87.4875) (width 0.25) (layer "F.Cu") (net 1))
 (segment (start 103.4 90.6) (end 109 90.6) (width 0.25) (layer "F.Cu") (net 1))
 (segment (start 97.374511 93.704511) (end 97.504511 93.704511) (width 0.25) (layer "F.Cu") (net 1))
 (segment (start 118.2 83.4) (end 118.225 83.375) (width 0.25) (layer "F.Cu") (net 1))
 (segment (start 102.8 91.6) (end 102.8 91.2) (width 0.25) (layer "F.Cu") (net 1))
 (segment (start 115 95) (end 115.25 94.75) (width 0.25) (layer "F.Cu") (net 1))
 (segment (start 126.1 94.875978) (end 126.1 95.74) (width 0.25) (layer "F.Cu") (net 1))
 (segment (start 117.6 91.4) (end 118.2 90.8) (width 0.25) (layer "F.Cu") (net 1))
 (segment (start 115.525 93.2375) (end 115.525 91.525) (width 0.25) (layer "F.Cu") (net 1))
 (segment (start 97.3 93.03) (end 97.3 93.63) (width 0.25) (layer "F.Cu") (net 1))
 (segment (start 122.024022 90.8) (end 126.1 94.875978) (width 0.25) (layer "F.Cu") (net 1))
 (segment (start 118.2 90.8) (end 122.024022 90.8) (width 0.25) (layer "F.Cu") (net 1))
 (segment (start 110.65 92.25) (end 109 90.6) (width 0.25) (layer "F.Cu") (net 1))
 (segment (start 109 90.6) (end 109 86.0875) (width 0.25) (layer "F.Cu") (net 1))
 (segment (start 100.3 92.1) (end 100.3 93.03) (width 0.25) (layer "F.Cu") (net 1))
 (segment (start 102.8 91.2) (end 103.4 90.6) (width 0.25) (layer "F.Cu") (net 1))
 (segment (start 110.8 95) (end 115 95) (width 0.25) (layer "F.Cu") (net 1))
 (segment (start 97.504511 93.704511) (end 97.6 93.8) (width 0.25) (layer "F.Cu") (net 1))
 (segment (start 100.3 93.5) (end 100.05 93.75) (width 0.25) (layer "F.Cu") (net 1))
 (segment (start 115.25 93.2375) (end 115.525 93.2375) (width 0.25) (layer "F.Cu") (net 1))
 (segment (start 118.225 83.375) (end 122.8 83.375) (width 0.25) (layer "F.Cu") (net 1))
 (via (at 102.8 91.6) (size 0.8) (drill 0.4) (layers "F.Cu" "B.Cu") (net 1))
 (via (at 100.2 92) (size 0.8) (drill 0.4) (layers "F.Cu" "B.Cu") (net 1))
 (via (at 117.6 91.4) (size 0.8) (drill 0.4) (layers "F.Cu" "B.Cu") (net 1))
 (via (at 97.3 91.9) (size 0.8) (drill 0.4) (layers "F.Cu" "B.Cu") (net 1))
 (via (at 115.525 91.525) (size 0.8) (drill 0.4) (layers "F.Cu" "B.Cu") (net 1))
 (segment (start 115.65 91.4) (end 117.6 91.4) (width 0.25) (layer "B.Cu") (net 1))
 (segment (start 100.2 92) (end 102.4 92) (width 0.25) (layer "B.Cu") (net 1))
 (segment (start 97.3 91.9) (end 97.4 92) (width 0.25) (layer "B.Cu") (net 1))
 (segment (start 115.525 91.525) (end 115.65 91.4) (width 0.25) (layer "B.Cu") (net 1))
 (segment (start 97.4 92) (end 100.2 92) (width 0.25) (layer "B.Cu") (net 1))
 (segment (start 102.4 92) (end 102.8 91.6) (width 0.25) (layer "B.Cu") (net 1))
 (segment (start 99.3 93.03) (end 99.3 84.96) (width 0.25) (layer "F.Cu") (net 8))
 (segment (start 99.3 84.96) (end 97.74 83.4) (width 0.25) (layer "F.Cu") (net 8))
 (segment (start 98.3 93.03) (end 98.3 85.9) (width 0.25) (layer "F.Cu") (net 7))
 (segment (start 96.4 84) (end 96.4 82.2) (width 0.25) (layer "F.Cu") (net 7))
 (segment (start 98.3 85.9) (end 96.4 84) (width 0.25) (layer "F.Cu") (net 7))
 (segment (start 96.4 82.2) (end 98.8 82.2) (width 0.25) (layer "F.Cu") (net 7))
 (segment (start 98.8 82.2) (end 100 83.4) (width 0.25) (layer "F.Cu") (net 7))
 (segment (start 100 83.4) (end 100.28 83.4) (width 0.25) (layer "F.Cu") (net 7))
 (segment (start 113.2 86.3755) (end 113.2 85.035) (width 0.25) (layer "F.Cu") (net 12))
 (segment (start 113.2 85.035) (end 111.54 83.375) (width 0.25) (layer "F.Cu") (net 12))
 (segment (start 113.2 93.2375) (end 113.2 91.4) (width 0.25) (layer "F.Cu") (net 12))
 (via (at 113.2 86.3755) (size 0.8) (drill 0.4) (layers "F.Cu" "B.Cu") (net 12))
 (via (at 113.2 91.4) (size 0.8) (drill 0.4) (layers "F.Cu" "B.Cu") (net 12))
 (segment (start 113.2 91.4) (end 113.2 86.3755) (width 0.25) (layer "B.Cu") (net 12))
 (segment (start 114 82.2) (end 114.08 82.28) (width 0.25) (layer "F.Cu") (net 11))
 (segment (start 110.365489 85.940989) (end 110.365489 82.234511) (width 0.25) (layer "F.Cu") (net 11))
 (segment (start 110.4 82.2) (end 114 82.2) (width 0.25) (layer "F.Cu") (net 11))
 (segment (start 110.8 86.3755) (end 110.365489 85.940989) (width 0.25) (layer "F.Cu") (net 11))
 (segment (start 112.7 92.3) (end 111.8 91.4) (width 0.25) (layer "F.Cu") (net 11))
 (segment (start 112.7 93.2375) (end 112.7 92.3) (width 0.25) (layer "F.Cu") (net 11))
 (segment (start 110.365489 82.234511) (end 110.4 82.2) (width 0.25) (layer "F.Cu") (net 11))
 (segment (start 114.08 82.28) (end 114.08 83.375) (width 0.25) (layer "F.Cu") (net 11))
 (via (at 110.8 86.3755) (size 0.8) (drill 0.4) (layers "F.Cu" "B.Cu") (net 11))
 (via (at 111.8 91.4) (size 0.8) (drill 0.4) (layers "F.Cu" "B.Cu") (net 11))
 (segment (start 110.8 90.4) (end 110.8 86.3755) (width 0.25) (layer "B.Cu") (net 11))
 (segment (start 111.8 91.4) (end 110.8 90.4) (width 0.25) (layer "B.Cu") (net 11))
 (segment (start 126.505 82) (end 127.88 83.375) (width 0.25) (layer "F.Cu") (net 2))
 (segment (start 124 85.6) (end 124 82) (width 0.25) (layer "F.Cu") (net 2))
 (segment (start 126.75 95.74) (end 126.75 88.35) (width 0.25) (layer "F.Cu") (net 2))
 (segment (start 124 82) (end 126.505 82) (width 0.25) (layer "F.Cu") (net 2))
 (segment (start 126.75 88.35) (end 124 85.6) (width 0.25) (layer "F.Cu") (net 2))
 (segment (start 127.4 95.74) (end 127.4 85.435) (width 0.25) (layer "F.Cu") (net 3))
 (segment (start 127.4 85.435) (end 125.34 83.375) (width 0.25) (layer "F.Cu") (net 3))
 (segment (start 110.4 89.3125) (end 112.775 89.3125) (width 0.25) (layer "F.Cu") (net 14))
 (segment (start 112.775 89.3125) (end 112.8 89.3375) (width 0.25) (layer "F.Cu") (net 14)))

